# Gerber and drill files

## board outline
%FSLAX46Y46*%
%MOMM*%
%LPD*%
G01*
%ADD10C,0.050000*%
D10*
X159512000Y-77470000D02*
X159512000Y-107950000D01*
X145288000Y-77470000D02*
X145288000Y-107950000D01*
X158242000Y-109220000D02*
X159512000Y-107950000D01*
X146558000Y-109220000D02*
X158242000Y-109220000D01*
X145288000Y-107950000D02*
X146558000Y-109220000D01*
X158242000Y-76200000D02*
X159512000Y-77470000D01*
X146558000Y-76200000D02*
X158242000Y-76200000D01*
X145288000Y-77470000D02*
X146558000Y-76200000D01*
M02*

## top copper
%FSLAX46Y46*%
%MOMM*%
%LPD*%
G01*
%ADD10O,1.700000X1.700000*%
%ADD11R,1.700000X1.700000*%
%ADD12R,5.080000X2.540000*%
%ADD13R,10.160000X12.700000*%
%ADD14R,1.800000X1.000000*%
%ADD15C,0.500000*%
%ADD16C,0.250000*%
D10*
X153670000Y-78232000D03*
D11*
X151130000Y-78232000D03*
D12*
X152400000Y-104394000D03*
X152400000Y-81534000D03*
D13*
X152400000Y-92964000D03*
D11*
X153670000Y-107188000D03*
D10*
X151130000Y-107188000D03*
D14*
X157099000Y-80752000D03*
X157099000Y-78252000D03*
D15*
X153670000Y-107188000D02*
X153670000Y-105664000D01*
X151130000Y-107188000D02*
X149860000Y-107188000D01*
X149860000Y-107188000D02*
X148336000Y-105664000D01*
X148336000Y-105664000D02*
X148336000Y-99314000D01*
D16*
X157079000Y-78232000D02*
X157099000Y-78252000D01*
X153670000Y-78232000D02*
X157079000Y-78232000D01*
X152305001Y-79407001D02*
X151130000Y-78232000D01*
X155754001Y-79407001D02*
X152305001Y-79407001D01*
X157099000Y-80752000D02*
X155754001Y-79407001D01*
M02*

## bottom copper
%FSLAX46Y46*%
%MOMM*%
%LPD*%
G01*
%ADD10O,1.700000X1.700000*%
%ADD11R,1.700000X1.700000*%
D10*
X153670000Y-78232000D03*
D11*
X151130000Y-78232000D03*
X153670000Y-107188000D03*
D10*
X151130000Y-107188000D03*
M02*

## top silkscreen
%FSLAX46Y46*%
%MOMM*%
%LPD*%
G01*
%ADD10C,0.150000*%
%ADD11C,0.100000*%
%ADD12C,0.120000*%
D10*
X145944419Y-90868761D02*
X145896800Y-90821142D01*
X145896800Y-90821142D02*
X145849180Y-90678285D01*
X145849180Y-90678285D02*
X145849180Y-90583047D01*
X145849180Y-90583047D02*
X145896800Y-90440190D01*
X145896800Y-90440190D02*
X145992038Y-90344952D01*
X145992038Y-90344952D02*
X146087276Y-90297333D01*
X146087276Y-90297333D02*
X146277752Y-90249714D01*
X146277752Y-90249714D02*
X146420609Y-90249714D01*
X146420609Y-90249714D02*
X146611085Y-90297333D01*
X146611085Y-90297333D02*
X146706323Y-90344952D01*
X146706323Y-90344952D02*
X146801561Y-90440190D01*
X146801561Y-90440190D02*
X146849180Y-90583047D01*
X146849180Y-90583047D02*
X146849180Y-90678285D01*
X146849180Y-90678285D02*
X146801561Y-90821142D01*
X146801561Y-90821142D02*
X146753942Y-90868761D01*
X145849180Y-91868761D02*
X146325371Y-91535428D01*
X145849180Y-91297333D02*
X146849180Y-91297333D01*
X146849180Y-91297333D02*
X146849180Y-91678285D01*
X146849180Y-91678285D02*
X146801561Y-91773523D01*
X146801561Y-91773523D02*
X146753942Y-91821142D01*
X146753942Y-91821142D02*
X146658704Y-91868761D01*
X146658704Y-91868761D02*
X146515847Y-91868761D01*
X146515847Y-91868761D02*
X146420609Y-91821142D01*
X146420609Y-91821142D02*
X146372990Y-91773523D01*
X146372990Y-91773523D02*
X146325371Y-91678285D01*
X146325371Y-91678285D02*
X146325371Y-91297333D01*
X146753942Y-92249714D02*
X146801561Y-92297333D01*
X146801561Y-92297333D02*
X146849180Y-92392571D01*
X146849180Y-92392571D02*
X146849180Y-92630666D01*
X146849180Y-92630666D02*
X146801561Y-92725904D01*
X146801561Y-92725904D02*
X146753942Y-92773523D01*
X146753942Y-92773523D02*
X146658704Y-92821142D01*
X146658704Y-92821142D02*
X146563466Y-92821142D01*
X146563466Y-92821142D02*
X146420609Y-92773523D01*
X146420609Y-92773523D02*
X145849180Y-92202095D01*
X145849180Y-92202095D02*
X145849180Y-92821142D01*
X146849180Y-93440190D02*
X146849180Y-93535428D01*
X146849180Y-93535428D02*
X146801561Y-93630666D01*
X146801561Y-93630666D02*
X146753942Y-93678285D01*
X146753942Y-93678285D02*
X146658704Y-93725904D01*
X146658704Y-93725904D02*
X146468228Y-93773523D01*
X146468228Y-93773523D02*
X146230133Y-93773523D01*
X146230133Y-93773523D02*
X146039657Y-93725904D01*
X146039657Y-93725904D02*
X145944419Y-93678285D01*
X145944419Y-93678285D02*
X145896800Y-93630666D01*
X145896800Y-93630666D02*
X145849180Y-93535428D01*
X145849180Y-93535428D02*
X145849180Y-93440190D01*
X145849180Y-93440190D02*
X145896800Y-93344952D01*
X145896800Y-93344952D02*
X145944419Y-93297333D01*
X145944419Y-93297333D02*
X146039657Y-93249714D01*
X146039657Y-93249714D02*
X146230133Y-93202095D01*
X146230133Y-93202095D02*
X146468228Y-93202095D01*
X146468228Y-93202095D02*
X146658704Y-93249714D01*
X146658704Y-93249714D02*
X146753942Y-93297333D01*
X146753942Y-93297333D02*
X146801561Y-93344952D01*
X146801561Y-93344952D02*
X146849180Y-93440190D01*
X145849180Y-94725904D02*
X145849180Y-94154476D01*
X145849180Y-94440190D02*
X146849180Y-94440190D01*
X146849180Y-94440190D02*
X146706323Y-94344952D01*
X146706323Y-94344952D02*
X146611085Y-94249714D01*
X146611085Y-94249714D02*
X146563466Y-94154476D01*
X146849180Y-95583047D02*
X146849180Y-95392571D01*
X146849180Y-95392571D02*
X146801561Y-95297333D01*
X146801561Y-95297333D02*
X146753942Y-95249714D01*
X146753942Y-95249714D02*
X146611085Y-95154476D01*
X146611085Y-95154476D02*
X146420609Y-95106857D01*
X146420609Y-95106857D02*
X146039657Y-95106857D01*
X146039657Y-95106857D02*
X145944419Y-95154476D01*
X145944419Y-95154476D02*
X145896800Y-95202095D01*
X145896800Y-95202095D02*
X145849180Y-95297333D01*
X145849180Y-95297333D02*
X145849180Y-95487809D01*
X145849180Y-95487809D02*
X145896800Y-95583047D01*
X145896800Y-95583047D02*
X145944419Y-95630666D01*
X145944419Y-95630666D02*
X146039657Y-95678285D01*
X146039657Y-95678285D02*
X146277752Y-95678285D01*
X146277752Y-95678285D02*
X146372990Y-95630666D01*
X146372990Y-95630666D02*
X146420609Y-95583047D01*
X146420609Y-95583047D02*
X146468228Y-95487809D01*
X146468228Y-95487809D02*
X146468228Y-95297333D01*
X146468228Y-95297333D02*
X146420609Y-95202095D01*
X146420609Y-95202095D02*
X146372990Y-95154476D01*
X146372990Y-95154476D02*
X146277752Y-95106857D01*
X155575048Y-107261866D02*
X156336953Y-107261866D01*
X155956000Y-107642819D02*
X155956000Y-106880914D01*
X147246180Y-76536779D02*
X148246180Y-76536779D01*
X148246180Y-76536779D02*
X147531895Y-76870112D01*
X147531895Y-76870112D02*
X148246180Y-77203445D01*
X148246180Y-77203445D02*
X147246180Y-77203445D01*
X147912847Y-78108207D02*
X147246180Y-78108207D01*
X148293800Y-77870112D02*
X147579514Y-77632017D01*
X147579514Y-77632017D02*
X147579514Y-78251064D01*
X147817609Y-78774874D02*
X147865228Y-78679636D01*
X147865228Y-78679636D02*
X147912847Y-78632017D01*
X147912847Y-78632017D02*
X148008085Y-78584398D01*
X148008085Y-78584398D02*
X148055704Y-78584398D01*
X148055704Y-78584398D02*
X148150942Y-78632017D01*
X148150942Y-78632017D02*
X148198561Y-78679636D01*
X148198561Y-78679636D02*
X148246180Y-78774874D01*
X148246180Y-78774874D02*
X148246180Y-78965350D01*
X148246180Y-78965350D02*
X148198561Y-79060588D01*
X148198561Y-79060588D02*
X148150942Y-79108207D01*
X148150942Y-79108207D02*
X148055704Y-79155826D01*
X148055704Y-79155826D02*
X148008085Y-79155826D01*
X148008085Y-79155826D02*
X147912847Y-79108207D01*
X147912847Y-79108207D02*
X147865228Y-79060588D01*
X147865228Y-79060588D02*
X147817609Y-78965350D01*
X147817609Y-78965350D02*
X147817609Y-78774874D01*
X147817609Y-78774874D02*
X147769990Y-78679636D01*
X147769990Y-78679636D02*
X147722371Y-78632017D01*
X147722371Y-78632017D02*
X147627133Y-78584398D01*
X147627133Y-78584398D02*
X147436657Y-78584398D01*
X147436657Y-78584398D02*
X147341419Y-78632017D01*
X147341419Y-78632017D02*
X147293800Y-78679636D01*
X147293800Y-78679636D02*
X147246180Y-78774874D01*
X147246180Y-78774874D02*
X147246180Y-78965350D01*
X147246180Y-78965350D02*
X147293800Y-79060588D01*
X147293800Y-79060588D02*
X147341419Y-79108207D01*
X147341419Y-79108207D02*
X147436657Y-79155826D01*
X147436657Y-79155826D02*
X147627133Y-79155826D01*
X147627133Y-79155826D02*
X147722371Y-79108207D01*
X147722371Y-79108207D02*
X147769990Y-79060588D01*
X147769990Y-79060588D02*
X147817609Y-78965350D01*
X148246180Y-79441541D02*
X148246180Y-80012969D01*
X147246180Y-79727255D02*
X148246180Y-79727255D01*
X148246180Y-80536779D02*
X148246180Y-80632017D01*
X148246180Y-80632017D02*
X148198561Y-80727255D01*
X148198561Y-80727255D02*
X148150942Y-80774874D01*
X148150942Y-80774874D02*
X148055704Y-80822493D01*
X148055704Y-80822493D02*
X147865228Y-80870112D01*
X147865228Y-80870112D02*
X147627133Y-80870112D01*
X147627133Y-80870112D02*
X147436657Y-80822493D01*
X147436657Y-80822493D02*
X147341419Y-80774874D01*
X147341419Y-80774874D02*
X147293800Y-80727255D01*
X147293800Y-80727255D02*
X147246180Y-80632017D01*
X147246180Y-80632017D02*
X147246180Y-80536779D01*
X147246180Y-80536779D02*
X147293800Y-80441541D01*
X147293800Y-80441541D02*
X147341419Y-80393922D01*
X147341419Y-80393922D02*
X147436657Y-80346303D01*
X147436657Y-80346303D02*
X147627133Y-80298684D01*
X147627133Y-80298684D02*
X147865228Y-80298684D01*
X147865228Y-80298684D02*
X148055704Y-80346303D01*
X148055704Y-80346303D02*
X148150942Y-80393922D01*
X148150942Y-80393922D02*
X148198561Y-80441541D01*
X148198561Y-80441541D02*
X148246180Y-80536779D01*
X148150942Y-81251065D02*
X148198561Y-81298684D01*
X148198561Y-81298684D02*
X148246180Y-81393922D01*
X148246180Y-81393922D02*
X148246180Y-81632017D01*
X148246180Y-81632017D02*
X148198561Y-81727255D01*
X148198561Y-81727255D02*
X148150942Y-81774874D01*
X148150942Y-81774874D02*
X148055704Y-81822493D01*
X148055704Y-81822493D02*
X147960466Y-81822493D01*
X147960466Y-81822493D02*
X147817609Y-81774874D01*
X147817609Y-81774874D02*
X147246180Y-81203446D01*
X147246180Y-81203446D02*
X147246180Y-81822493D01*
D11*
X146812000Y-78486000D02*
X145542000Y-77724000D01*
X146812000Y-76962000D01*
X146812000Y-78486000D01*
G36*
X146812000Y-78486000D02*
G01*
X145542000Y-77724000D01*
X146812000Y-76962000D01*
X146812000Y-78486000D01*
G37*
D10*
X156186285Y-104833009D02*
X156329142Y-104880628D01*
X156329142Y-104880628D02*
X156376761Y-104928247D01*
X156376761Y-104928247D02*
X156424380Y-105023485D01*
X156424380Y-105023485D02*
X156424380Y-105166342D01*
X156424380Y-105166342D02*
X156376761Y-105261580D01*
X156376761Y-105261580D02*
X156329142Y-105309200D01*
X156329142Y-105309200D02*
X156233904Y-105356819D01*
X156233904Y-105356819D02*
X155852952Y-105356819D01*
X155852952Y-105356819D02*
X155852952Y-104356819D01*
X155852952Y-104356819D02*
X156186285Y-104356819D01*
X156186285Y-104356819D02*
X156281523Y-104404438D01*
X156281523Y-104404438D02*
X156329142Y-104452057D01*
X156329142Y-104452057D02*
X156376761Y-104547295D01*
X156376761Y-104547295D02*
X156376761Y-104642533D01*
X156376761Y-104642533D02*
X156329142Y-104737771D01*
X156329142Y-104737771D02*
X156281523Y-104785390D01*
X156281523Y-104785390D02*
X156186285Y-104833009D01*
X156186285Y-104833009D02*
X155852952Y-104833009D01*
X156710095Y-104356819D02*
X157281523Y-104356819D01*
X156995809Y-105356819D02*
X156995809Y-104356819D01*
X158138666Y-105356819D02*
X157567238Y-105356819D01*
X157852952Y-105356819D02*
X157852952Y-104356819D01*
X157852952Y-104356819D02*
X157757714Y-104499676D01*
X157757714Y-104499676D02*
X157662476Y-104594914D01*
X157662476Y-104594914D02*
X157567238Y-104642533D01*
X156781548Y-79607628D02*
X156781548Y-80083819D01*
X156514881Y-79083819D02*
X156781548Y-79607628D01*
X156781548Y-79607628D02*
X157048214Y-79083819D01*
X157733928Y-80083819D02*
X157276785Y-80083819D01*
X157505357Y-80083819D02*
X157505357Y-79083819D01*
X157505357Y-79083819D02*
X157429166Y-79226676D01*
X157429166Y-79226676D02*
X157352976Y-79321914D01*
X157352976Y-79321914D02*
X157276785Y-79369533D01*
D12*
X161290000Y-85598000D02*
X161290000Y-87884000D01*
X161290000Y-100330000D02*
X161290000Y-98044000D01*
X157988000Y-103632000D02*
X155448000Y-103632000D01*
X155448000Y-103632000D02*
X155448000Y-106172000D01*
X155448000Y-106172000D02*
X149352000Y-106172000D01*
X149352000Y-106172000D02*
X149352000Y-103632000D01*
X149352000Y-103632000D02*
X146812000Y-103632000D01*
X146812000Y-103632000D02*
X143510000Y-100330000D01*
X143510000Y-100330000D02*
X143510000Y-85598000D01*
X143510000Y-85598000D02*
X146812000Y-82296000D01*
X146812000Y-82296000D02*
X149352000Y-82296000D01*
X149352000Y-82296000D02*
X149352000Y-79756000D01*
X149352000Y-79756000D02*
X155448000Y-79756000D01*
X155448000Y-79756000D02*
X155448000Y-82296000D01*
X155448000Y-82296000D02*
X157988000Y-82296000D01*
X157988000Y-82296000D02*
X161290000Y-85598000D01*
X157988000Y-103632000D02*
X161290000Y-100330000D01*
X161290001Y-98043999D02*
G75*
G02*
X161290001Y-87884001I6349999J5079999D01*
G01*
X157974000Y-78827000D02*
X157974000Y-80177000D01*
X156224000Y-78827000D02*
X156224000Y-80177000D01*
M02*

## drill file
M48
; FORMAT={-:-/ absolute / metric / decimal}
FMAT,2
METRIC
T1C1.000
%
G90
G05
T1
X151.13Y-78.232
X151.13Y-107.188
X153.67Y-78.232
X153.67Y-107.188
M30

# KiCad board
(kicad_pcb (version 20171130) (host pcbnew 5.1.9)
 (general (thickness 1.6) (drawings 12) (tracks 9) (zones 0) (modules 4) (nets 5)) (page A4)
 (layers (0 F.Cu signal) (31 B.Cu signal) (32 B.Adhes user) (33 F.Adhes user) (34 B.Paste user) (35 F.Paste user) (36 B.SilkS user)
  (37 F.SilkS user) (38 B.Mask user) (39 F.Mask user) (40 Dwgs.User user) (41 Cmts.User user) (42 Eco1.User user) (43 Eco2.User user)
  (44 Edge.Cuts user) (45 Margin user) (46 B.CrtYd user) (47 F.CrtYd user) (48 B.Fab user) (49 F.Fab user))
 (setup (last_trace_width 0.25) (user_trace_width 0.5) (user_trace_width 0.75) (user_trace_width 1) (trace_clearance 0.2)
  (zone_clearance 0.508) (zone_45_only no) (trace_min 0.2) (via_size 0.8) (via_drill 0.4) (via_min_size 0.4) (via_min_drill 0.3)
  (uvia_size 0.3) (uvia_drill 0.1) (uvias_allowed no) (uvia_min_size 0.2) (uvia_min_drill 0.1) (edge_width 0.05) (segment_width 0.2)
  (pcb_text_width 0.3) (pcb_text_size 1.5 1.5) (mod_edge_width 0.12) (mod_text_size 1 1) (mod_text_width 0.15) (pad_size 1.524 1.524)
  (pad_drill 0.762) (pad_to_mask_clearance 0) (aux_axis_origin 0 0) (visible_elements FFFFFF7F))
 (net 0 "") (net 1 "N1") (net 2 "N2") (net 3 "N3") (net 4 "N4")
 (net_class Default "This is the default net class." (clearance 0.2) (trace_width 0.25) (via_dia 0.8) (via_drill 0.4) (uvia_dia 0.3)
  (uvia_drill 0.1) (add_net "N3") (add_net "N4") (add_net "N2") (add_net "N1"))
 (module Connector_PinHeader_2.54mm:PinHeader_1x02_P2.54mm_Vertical (layer B.Cu) (at 151.13 78.232 270)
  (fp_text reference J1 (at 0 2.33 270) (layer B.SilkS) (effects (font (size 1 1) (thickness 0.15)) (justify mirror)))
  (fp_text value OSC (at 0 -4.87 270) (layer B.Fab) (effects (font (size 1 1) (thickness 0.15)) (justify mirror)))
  (pad 2 thru_hole oval (at 0 -2.54 270) (size 1.7 1.7) (drill 1) (layers *.Cu *.Mask) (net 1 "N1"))
  (pad 1 thru_hole rect (at 0 0 270) (size 1.7 1.7) (drill 1) (layers *.Cu *.Mask) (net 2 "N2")))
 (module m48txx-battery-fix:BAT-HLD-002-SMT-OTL (layer F.Cu) (at 152.4 92.964 90)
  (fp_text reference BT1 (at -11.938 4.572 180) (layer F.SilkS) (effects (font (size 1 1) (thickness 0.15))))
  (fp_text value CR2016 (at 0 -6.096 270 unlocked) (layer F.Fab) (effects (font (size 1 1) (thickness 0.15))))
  (fp_line (start 7.366 8.89) (end 5.08 8.89) (layer F.SilkS) (width 0.12))
  (fp_line (start -7.366 8.89) (end -5.08 8.89) (layer F.SilkS) (width 0.12))
  (fp_line (start -10.668 5.588) (end -10.668 3.048) (layer F.SilkS) (width 0.12))
  (fp_line (start -10.668 3.048) (end -13.208 3.048) (layer F.SilkS) (width 0.12))
  (fp_line (start -13.208 3.048) (end -13.208 -3.048) (layer F.SilkS) (width 0.12))
  (fp_line (start -13.208 -3.048) (end -10.668 -3.048) (layer F.SilkS) (width 0.12))
  (fp_line (start -10.668 -3.048) (end -10.668 -5.588) (layer F.SilkS) (width 0.12))
  (fp_line (start -10.668 -5.588) (end -7.366 -8.89) (layer F.SilkS) (width 0.12))
  (fp_line (start -7.366 -8.89) (end 7.366 -8.89) (layer F.SilkS) (width 0.12))
  (fp_line (start 7.366 -8.89) (end 10.668 -5.588) (layer F.SilkS) (width 0.12))
  (fp_line (start 10.668 -5.588) (end 10.668 -3.048) (layer F.SilkS) (width 0.12))
  (fp_line (start 10.668 -3.048) (end 13.208 -3.048) (layer F.SilkS) (width 0.12))
  (fp_line (start 13.208 -3.048) (end 13.208 3.048) (layer F.SilkS) (width 0.12))
  (fp_line (start 13.208 3.048) (end 10.668 3.048) (layer F.SilkS) (width 0.12))
  (fp_line (start 10.668 3.048) (end 10.668 5.588) (layer F.SilkS) (width 0.12))
  (fp_line (start 10.668 5.588) (end 7.366 8.89) (layer F.SilkS) (width 0.12))
  (fp_line (start -10.668 5.588) (end -7.366 8.89) (layer F.SilkS) (width 0.12))
  (fp_arc (start 0 15.24) (end 5.079999 8.890001) (angle -77.31961651) (layer F.SilkS) (width 0.12))
  (pad 1 smd rect (at -12.7 0 90) (size 2.54 5.08) (drill (offset 1.27 0)) (layers F.Cu F.Paste F.Mask) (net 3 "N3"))
  (pad 1 smd rect (at 12.7 0 90) (size 2.54 5.08) (drill (offset -1.27 0)) (layers F.Cu F.Paste F.Mask) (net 3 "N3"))
  (pad 2 smd rect (at 0 0 90) (size 12.7 10.16) (layers F.Cu F.Mask) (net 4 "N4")))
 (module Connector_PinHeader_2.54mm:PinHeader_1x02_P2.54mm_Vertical (layer B.Cu) (at 153.67 107.188 90)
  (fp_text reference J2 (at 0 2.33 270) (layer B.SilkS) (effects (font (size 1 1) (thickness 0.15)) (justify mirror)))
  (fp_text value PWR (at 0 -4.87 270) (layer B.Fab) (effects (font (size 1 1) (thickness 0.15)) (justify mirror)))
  (pad 1 thru_hole rect (at 0 0 90) (size 1.7 1.7) (drill 1) (layers *.Cu *.Mask) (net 3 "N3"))
  (pad 2 thru_hole oval (at 0 -2.54 90) (size 1.7 1.7) (drill 1) (layers *.Cu *.Mask) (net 4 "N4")))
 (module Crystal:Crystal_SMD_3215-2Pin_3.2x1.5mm (layer F.Cu) (at 157.099 79.502 270)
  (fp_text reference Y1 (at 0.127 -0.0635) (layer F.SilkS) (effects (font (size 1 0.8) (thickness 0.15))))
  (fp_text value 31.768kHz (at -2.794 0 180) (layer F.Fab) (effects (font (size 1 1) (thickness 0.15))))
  (fp_line (start -0.675 -0.875) (end 0.675 -0.875) (layer F.SilkS) (width 0.12))
  (fp_line (start -0.675 0.875) (end 0.675 0.875) (layer F.SilkS) (width 0.12))
  (pad 1 smd rect (at 1.25 0 270) (size 1 1.8) (layers F.Cu F.Paste F.Mask) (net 2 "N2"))
  (pad 2 smd rect (at -1.25 0 270) (size 1 1.8) (layers F.Cu F.Paste F.Mask) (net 1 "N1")))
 (gr_line (start 159.512 77.47) (end 159.512 107.95) (layer Edge.Cuts) (width 0.05))
 (gr_line (start 145.288 77.47) (end 145.288 107.95) (layer Edge.Cuts) (width 0.05))
 (gr_line (start 158.242 109.22) (end 159.512 107.95) (layer Edge.Cuts) (width 0.05))
 (gr_line (start 146.558 109.22) (end 158.242 109.22) (layer Edge.Cuts) (width 0.05))
 (gr_line (start 145.288 107.95) (end 146.558 109.22) (layer Edge.Cuts) (width 0.05))
 (gr_line (start 158.242 76.2) (end 159.512 77.47) (layer Edge.Cuts) (width 0.05))
 (gr_line (start 146.558 76.2) (end 158.242 76.2) (layer Edge.Cuts) (width 0.05))
 (gr_line (start 145.288 77.47) (end 146.558 76.2) (layer Edge.Cuts) (width 0.05))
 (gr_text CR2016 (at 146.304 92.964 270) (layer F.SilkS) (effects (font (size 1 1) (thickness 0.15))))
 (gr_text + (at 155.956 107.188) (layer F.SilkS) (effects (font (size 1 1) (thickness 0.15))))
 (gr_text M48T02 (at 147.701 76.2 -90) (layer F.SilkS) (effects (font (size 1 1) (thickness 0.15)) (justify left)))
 (gr_poly (pts (xy 146.812 78.486) (xy 145.542 77.724) (xy 146.812 76.962)) (layer F.SilkS) (width 0.1))
 (segment (start 153.67 107.188) (end 153.67 105.664) (width 0.5) (layer F.Cu) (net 3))
 (segment (start 151.13 107.188) (end 149.86 107.188) (width 0.5) (layer F.Cu) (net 4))
 (segment (start 149.86 107.188) (end 148.336 105.664) (width 0.5) (layer F.Cu) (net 4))
 (segment (start 148.336 105.664) (end 148.336 99.314) (width 0.5) (layer F.Cu) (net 4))
 (segment (start 157.079 78.232) (end 157.099 78.252) (width 0.25) (layer F.Cu) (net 1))
 (segment (start 153.67 78.232) (end 157.079 78.232) (width 0.25) (layer F.Cu) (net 1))
 (segment (start 152.305001 79.407001) (end 151.13 78.232) (width 0.25) (layer F.Cu) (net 2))
 (segment (start 155.754001 79.407001) (end 152.305001 79.407001) (width 0.25) (layer F.Cu) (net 2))
 (segment (start 157.099 80.752) (end 155.754001 79.407001) (width 0.25) (layer F.Cu) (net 2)))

